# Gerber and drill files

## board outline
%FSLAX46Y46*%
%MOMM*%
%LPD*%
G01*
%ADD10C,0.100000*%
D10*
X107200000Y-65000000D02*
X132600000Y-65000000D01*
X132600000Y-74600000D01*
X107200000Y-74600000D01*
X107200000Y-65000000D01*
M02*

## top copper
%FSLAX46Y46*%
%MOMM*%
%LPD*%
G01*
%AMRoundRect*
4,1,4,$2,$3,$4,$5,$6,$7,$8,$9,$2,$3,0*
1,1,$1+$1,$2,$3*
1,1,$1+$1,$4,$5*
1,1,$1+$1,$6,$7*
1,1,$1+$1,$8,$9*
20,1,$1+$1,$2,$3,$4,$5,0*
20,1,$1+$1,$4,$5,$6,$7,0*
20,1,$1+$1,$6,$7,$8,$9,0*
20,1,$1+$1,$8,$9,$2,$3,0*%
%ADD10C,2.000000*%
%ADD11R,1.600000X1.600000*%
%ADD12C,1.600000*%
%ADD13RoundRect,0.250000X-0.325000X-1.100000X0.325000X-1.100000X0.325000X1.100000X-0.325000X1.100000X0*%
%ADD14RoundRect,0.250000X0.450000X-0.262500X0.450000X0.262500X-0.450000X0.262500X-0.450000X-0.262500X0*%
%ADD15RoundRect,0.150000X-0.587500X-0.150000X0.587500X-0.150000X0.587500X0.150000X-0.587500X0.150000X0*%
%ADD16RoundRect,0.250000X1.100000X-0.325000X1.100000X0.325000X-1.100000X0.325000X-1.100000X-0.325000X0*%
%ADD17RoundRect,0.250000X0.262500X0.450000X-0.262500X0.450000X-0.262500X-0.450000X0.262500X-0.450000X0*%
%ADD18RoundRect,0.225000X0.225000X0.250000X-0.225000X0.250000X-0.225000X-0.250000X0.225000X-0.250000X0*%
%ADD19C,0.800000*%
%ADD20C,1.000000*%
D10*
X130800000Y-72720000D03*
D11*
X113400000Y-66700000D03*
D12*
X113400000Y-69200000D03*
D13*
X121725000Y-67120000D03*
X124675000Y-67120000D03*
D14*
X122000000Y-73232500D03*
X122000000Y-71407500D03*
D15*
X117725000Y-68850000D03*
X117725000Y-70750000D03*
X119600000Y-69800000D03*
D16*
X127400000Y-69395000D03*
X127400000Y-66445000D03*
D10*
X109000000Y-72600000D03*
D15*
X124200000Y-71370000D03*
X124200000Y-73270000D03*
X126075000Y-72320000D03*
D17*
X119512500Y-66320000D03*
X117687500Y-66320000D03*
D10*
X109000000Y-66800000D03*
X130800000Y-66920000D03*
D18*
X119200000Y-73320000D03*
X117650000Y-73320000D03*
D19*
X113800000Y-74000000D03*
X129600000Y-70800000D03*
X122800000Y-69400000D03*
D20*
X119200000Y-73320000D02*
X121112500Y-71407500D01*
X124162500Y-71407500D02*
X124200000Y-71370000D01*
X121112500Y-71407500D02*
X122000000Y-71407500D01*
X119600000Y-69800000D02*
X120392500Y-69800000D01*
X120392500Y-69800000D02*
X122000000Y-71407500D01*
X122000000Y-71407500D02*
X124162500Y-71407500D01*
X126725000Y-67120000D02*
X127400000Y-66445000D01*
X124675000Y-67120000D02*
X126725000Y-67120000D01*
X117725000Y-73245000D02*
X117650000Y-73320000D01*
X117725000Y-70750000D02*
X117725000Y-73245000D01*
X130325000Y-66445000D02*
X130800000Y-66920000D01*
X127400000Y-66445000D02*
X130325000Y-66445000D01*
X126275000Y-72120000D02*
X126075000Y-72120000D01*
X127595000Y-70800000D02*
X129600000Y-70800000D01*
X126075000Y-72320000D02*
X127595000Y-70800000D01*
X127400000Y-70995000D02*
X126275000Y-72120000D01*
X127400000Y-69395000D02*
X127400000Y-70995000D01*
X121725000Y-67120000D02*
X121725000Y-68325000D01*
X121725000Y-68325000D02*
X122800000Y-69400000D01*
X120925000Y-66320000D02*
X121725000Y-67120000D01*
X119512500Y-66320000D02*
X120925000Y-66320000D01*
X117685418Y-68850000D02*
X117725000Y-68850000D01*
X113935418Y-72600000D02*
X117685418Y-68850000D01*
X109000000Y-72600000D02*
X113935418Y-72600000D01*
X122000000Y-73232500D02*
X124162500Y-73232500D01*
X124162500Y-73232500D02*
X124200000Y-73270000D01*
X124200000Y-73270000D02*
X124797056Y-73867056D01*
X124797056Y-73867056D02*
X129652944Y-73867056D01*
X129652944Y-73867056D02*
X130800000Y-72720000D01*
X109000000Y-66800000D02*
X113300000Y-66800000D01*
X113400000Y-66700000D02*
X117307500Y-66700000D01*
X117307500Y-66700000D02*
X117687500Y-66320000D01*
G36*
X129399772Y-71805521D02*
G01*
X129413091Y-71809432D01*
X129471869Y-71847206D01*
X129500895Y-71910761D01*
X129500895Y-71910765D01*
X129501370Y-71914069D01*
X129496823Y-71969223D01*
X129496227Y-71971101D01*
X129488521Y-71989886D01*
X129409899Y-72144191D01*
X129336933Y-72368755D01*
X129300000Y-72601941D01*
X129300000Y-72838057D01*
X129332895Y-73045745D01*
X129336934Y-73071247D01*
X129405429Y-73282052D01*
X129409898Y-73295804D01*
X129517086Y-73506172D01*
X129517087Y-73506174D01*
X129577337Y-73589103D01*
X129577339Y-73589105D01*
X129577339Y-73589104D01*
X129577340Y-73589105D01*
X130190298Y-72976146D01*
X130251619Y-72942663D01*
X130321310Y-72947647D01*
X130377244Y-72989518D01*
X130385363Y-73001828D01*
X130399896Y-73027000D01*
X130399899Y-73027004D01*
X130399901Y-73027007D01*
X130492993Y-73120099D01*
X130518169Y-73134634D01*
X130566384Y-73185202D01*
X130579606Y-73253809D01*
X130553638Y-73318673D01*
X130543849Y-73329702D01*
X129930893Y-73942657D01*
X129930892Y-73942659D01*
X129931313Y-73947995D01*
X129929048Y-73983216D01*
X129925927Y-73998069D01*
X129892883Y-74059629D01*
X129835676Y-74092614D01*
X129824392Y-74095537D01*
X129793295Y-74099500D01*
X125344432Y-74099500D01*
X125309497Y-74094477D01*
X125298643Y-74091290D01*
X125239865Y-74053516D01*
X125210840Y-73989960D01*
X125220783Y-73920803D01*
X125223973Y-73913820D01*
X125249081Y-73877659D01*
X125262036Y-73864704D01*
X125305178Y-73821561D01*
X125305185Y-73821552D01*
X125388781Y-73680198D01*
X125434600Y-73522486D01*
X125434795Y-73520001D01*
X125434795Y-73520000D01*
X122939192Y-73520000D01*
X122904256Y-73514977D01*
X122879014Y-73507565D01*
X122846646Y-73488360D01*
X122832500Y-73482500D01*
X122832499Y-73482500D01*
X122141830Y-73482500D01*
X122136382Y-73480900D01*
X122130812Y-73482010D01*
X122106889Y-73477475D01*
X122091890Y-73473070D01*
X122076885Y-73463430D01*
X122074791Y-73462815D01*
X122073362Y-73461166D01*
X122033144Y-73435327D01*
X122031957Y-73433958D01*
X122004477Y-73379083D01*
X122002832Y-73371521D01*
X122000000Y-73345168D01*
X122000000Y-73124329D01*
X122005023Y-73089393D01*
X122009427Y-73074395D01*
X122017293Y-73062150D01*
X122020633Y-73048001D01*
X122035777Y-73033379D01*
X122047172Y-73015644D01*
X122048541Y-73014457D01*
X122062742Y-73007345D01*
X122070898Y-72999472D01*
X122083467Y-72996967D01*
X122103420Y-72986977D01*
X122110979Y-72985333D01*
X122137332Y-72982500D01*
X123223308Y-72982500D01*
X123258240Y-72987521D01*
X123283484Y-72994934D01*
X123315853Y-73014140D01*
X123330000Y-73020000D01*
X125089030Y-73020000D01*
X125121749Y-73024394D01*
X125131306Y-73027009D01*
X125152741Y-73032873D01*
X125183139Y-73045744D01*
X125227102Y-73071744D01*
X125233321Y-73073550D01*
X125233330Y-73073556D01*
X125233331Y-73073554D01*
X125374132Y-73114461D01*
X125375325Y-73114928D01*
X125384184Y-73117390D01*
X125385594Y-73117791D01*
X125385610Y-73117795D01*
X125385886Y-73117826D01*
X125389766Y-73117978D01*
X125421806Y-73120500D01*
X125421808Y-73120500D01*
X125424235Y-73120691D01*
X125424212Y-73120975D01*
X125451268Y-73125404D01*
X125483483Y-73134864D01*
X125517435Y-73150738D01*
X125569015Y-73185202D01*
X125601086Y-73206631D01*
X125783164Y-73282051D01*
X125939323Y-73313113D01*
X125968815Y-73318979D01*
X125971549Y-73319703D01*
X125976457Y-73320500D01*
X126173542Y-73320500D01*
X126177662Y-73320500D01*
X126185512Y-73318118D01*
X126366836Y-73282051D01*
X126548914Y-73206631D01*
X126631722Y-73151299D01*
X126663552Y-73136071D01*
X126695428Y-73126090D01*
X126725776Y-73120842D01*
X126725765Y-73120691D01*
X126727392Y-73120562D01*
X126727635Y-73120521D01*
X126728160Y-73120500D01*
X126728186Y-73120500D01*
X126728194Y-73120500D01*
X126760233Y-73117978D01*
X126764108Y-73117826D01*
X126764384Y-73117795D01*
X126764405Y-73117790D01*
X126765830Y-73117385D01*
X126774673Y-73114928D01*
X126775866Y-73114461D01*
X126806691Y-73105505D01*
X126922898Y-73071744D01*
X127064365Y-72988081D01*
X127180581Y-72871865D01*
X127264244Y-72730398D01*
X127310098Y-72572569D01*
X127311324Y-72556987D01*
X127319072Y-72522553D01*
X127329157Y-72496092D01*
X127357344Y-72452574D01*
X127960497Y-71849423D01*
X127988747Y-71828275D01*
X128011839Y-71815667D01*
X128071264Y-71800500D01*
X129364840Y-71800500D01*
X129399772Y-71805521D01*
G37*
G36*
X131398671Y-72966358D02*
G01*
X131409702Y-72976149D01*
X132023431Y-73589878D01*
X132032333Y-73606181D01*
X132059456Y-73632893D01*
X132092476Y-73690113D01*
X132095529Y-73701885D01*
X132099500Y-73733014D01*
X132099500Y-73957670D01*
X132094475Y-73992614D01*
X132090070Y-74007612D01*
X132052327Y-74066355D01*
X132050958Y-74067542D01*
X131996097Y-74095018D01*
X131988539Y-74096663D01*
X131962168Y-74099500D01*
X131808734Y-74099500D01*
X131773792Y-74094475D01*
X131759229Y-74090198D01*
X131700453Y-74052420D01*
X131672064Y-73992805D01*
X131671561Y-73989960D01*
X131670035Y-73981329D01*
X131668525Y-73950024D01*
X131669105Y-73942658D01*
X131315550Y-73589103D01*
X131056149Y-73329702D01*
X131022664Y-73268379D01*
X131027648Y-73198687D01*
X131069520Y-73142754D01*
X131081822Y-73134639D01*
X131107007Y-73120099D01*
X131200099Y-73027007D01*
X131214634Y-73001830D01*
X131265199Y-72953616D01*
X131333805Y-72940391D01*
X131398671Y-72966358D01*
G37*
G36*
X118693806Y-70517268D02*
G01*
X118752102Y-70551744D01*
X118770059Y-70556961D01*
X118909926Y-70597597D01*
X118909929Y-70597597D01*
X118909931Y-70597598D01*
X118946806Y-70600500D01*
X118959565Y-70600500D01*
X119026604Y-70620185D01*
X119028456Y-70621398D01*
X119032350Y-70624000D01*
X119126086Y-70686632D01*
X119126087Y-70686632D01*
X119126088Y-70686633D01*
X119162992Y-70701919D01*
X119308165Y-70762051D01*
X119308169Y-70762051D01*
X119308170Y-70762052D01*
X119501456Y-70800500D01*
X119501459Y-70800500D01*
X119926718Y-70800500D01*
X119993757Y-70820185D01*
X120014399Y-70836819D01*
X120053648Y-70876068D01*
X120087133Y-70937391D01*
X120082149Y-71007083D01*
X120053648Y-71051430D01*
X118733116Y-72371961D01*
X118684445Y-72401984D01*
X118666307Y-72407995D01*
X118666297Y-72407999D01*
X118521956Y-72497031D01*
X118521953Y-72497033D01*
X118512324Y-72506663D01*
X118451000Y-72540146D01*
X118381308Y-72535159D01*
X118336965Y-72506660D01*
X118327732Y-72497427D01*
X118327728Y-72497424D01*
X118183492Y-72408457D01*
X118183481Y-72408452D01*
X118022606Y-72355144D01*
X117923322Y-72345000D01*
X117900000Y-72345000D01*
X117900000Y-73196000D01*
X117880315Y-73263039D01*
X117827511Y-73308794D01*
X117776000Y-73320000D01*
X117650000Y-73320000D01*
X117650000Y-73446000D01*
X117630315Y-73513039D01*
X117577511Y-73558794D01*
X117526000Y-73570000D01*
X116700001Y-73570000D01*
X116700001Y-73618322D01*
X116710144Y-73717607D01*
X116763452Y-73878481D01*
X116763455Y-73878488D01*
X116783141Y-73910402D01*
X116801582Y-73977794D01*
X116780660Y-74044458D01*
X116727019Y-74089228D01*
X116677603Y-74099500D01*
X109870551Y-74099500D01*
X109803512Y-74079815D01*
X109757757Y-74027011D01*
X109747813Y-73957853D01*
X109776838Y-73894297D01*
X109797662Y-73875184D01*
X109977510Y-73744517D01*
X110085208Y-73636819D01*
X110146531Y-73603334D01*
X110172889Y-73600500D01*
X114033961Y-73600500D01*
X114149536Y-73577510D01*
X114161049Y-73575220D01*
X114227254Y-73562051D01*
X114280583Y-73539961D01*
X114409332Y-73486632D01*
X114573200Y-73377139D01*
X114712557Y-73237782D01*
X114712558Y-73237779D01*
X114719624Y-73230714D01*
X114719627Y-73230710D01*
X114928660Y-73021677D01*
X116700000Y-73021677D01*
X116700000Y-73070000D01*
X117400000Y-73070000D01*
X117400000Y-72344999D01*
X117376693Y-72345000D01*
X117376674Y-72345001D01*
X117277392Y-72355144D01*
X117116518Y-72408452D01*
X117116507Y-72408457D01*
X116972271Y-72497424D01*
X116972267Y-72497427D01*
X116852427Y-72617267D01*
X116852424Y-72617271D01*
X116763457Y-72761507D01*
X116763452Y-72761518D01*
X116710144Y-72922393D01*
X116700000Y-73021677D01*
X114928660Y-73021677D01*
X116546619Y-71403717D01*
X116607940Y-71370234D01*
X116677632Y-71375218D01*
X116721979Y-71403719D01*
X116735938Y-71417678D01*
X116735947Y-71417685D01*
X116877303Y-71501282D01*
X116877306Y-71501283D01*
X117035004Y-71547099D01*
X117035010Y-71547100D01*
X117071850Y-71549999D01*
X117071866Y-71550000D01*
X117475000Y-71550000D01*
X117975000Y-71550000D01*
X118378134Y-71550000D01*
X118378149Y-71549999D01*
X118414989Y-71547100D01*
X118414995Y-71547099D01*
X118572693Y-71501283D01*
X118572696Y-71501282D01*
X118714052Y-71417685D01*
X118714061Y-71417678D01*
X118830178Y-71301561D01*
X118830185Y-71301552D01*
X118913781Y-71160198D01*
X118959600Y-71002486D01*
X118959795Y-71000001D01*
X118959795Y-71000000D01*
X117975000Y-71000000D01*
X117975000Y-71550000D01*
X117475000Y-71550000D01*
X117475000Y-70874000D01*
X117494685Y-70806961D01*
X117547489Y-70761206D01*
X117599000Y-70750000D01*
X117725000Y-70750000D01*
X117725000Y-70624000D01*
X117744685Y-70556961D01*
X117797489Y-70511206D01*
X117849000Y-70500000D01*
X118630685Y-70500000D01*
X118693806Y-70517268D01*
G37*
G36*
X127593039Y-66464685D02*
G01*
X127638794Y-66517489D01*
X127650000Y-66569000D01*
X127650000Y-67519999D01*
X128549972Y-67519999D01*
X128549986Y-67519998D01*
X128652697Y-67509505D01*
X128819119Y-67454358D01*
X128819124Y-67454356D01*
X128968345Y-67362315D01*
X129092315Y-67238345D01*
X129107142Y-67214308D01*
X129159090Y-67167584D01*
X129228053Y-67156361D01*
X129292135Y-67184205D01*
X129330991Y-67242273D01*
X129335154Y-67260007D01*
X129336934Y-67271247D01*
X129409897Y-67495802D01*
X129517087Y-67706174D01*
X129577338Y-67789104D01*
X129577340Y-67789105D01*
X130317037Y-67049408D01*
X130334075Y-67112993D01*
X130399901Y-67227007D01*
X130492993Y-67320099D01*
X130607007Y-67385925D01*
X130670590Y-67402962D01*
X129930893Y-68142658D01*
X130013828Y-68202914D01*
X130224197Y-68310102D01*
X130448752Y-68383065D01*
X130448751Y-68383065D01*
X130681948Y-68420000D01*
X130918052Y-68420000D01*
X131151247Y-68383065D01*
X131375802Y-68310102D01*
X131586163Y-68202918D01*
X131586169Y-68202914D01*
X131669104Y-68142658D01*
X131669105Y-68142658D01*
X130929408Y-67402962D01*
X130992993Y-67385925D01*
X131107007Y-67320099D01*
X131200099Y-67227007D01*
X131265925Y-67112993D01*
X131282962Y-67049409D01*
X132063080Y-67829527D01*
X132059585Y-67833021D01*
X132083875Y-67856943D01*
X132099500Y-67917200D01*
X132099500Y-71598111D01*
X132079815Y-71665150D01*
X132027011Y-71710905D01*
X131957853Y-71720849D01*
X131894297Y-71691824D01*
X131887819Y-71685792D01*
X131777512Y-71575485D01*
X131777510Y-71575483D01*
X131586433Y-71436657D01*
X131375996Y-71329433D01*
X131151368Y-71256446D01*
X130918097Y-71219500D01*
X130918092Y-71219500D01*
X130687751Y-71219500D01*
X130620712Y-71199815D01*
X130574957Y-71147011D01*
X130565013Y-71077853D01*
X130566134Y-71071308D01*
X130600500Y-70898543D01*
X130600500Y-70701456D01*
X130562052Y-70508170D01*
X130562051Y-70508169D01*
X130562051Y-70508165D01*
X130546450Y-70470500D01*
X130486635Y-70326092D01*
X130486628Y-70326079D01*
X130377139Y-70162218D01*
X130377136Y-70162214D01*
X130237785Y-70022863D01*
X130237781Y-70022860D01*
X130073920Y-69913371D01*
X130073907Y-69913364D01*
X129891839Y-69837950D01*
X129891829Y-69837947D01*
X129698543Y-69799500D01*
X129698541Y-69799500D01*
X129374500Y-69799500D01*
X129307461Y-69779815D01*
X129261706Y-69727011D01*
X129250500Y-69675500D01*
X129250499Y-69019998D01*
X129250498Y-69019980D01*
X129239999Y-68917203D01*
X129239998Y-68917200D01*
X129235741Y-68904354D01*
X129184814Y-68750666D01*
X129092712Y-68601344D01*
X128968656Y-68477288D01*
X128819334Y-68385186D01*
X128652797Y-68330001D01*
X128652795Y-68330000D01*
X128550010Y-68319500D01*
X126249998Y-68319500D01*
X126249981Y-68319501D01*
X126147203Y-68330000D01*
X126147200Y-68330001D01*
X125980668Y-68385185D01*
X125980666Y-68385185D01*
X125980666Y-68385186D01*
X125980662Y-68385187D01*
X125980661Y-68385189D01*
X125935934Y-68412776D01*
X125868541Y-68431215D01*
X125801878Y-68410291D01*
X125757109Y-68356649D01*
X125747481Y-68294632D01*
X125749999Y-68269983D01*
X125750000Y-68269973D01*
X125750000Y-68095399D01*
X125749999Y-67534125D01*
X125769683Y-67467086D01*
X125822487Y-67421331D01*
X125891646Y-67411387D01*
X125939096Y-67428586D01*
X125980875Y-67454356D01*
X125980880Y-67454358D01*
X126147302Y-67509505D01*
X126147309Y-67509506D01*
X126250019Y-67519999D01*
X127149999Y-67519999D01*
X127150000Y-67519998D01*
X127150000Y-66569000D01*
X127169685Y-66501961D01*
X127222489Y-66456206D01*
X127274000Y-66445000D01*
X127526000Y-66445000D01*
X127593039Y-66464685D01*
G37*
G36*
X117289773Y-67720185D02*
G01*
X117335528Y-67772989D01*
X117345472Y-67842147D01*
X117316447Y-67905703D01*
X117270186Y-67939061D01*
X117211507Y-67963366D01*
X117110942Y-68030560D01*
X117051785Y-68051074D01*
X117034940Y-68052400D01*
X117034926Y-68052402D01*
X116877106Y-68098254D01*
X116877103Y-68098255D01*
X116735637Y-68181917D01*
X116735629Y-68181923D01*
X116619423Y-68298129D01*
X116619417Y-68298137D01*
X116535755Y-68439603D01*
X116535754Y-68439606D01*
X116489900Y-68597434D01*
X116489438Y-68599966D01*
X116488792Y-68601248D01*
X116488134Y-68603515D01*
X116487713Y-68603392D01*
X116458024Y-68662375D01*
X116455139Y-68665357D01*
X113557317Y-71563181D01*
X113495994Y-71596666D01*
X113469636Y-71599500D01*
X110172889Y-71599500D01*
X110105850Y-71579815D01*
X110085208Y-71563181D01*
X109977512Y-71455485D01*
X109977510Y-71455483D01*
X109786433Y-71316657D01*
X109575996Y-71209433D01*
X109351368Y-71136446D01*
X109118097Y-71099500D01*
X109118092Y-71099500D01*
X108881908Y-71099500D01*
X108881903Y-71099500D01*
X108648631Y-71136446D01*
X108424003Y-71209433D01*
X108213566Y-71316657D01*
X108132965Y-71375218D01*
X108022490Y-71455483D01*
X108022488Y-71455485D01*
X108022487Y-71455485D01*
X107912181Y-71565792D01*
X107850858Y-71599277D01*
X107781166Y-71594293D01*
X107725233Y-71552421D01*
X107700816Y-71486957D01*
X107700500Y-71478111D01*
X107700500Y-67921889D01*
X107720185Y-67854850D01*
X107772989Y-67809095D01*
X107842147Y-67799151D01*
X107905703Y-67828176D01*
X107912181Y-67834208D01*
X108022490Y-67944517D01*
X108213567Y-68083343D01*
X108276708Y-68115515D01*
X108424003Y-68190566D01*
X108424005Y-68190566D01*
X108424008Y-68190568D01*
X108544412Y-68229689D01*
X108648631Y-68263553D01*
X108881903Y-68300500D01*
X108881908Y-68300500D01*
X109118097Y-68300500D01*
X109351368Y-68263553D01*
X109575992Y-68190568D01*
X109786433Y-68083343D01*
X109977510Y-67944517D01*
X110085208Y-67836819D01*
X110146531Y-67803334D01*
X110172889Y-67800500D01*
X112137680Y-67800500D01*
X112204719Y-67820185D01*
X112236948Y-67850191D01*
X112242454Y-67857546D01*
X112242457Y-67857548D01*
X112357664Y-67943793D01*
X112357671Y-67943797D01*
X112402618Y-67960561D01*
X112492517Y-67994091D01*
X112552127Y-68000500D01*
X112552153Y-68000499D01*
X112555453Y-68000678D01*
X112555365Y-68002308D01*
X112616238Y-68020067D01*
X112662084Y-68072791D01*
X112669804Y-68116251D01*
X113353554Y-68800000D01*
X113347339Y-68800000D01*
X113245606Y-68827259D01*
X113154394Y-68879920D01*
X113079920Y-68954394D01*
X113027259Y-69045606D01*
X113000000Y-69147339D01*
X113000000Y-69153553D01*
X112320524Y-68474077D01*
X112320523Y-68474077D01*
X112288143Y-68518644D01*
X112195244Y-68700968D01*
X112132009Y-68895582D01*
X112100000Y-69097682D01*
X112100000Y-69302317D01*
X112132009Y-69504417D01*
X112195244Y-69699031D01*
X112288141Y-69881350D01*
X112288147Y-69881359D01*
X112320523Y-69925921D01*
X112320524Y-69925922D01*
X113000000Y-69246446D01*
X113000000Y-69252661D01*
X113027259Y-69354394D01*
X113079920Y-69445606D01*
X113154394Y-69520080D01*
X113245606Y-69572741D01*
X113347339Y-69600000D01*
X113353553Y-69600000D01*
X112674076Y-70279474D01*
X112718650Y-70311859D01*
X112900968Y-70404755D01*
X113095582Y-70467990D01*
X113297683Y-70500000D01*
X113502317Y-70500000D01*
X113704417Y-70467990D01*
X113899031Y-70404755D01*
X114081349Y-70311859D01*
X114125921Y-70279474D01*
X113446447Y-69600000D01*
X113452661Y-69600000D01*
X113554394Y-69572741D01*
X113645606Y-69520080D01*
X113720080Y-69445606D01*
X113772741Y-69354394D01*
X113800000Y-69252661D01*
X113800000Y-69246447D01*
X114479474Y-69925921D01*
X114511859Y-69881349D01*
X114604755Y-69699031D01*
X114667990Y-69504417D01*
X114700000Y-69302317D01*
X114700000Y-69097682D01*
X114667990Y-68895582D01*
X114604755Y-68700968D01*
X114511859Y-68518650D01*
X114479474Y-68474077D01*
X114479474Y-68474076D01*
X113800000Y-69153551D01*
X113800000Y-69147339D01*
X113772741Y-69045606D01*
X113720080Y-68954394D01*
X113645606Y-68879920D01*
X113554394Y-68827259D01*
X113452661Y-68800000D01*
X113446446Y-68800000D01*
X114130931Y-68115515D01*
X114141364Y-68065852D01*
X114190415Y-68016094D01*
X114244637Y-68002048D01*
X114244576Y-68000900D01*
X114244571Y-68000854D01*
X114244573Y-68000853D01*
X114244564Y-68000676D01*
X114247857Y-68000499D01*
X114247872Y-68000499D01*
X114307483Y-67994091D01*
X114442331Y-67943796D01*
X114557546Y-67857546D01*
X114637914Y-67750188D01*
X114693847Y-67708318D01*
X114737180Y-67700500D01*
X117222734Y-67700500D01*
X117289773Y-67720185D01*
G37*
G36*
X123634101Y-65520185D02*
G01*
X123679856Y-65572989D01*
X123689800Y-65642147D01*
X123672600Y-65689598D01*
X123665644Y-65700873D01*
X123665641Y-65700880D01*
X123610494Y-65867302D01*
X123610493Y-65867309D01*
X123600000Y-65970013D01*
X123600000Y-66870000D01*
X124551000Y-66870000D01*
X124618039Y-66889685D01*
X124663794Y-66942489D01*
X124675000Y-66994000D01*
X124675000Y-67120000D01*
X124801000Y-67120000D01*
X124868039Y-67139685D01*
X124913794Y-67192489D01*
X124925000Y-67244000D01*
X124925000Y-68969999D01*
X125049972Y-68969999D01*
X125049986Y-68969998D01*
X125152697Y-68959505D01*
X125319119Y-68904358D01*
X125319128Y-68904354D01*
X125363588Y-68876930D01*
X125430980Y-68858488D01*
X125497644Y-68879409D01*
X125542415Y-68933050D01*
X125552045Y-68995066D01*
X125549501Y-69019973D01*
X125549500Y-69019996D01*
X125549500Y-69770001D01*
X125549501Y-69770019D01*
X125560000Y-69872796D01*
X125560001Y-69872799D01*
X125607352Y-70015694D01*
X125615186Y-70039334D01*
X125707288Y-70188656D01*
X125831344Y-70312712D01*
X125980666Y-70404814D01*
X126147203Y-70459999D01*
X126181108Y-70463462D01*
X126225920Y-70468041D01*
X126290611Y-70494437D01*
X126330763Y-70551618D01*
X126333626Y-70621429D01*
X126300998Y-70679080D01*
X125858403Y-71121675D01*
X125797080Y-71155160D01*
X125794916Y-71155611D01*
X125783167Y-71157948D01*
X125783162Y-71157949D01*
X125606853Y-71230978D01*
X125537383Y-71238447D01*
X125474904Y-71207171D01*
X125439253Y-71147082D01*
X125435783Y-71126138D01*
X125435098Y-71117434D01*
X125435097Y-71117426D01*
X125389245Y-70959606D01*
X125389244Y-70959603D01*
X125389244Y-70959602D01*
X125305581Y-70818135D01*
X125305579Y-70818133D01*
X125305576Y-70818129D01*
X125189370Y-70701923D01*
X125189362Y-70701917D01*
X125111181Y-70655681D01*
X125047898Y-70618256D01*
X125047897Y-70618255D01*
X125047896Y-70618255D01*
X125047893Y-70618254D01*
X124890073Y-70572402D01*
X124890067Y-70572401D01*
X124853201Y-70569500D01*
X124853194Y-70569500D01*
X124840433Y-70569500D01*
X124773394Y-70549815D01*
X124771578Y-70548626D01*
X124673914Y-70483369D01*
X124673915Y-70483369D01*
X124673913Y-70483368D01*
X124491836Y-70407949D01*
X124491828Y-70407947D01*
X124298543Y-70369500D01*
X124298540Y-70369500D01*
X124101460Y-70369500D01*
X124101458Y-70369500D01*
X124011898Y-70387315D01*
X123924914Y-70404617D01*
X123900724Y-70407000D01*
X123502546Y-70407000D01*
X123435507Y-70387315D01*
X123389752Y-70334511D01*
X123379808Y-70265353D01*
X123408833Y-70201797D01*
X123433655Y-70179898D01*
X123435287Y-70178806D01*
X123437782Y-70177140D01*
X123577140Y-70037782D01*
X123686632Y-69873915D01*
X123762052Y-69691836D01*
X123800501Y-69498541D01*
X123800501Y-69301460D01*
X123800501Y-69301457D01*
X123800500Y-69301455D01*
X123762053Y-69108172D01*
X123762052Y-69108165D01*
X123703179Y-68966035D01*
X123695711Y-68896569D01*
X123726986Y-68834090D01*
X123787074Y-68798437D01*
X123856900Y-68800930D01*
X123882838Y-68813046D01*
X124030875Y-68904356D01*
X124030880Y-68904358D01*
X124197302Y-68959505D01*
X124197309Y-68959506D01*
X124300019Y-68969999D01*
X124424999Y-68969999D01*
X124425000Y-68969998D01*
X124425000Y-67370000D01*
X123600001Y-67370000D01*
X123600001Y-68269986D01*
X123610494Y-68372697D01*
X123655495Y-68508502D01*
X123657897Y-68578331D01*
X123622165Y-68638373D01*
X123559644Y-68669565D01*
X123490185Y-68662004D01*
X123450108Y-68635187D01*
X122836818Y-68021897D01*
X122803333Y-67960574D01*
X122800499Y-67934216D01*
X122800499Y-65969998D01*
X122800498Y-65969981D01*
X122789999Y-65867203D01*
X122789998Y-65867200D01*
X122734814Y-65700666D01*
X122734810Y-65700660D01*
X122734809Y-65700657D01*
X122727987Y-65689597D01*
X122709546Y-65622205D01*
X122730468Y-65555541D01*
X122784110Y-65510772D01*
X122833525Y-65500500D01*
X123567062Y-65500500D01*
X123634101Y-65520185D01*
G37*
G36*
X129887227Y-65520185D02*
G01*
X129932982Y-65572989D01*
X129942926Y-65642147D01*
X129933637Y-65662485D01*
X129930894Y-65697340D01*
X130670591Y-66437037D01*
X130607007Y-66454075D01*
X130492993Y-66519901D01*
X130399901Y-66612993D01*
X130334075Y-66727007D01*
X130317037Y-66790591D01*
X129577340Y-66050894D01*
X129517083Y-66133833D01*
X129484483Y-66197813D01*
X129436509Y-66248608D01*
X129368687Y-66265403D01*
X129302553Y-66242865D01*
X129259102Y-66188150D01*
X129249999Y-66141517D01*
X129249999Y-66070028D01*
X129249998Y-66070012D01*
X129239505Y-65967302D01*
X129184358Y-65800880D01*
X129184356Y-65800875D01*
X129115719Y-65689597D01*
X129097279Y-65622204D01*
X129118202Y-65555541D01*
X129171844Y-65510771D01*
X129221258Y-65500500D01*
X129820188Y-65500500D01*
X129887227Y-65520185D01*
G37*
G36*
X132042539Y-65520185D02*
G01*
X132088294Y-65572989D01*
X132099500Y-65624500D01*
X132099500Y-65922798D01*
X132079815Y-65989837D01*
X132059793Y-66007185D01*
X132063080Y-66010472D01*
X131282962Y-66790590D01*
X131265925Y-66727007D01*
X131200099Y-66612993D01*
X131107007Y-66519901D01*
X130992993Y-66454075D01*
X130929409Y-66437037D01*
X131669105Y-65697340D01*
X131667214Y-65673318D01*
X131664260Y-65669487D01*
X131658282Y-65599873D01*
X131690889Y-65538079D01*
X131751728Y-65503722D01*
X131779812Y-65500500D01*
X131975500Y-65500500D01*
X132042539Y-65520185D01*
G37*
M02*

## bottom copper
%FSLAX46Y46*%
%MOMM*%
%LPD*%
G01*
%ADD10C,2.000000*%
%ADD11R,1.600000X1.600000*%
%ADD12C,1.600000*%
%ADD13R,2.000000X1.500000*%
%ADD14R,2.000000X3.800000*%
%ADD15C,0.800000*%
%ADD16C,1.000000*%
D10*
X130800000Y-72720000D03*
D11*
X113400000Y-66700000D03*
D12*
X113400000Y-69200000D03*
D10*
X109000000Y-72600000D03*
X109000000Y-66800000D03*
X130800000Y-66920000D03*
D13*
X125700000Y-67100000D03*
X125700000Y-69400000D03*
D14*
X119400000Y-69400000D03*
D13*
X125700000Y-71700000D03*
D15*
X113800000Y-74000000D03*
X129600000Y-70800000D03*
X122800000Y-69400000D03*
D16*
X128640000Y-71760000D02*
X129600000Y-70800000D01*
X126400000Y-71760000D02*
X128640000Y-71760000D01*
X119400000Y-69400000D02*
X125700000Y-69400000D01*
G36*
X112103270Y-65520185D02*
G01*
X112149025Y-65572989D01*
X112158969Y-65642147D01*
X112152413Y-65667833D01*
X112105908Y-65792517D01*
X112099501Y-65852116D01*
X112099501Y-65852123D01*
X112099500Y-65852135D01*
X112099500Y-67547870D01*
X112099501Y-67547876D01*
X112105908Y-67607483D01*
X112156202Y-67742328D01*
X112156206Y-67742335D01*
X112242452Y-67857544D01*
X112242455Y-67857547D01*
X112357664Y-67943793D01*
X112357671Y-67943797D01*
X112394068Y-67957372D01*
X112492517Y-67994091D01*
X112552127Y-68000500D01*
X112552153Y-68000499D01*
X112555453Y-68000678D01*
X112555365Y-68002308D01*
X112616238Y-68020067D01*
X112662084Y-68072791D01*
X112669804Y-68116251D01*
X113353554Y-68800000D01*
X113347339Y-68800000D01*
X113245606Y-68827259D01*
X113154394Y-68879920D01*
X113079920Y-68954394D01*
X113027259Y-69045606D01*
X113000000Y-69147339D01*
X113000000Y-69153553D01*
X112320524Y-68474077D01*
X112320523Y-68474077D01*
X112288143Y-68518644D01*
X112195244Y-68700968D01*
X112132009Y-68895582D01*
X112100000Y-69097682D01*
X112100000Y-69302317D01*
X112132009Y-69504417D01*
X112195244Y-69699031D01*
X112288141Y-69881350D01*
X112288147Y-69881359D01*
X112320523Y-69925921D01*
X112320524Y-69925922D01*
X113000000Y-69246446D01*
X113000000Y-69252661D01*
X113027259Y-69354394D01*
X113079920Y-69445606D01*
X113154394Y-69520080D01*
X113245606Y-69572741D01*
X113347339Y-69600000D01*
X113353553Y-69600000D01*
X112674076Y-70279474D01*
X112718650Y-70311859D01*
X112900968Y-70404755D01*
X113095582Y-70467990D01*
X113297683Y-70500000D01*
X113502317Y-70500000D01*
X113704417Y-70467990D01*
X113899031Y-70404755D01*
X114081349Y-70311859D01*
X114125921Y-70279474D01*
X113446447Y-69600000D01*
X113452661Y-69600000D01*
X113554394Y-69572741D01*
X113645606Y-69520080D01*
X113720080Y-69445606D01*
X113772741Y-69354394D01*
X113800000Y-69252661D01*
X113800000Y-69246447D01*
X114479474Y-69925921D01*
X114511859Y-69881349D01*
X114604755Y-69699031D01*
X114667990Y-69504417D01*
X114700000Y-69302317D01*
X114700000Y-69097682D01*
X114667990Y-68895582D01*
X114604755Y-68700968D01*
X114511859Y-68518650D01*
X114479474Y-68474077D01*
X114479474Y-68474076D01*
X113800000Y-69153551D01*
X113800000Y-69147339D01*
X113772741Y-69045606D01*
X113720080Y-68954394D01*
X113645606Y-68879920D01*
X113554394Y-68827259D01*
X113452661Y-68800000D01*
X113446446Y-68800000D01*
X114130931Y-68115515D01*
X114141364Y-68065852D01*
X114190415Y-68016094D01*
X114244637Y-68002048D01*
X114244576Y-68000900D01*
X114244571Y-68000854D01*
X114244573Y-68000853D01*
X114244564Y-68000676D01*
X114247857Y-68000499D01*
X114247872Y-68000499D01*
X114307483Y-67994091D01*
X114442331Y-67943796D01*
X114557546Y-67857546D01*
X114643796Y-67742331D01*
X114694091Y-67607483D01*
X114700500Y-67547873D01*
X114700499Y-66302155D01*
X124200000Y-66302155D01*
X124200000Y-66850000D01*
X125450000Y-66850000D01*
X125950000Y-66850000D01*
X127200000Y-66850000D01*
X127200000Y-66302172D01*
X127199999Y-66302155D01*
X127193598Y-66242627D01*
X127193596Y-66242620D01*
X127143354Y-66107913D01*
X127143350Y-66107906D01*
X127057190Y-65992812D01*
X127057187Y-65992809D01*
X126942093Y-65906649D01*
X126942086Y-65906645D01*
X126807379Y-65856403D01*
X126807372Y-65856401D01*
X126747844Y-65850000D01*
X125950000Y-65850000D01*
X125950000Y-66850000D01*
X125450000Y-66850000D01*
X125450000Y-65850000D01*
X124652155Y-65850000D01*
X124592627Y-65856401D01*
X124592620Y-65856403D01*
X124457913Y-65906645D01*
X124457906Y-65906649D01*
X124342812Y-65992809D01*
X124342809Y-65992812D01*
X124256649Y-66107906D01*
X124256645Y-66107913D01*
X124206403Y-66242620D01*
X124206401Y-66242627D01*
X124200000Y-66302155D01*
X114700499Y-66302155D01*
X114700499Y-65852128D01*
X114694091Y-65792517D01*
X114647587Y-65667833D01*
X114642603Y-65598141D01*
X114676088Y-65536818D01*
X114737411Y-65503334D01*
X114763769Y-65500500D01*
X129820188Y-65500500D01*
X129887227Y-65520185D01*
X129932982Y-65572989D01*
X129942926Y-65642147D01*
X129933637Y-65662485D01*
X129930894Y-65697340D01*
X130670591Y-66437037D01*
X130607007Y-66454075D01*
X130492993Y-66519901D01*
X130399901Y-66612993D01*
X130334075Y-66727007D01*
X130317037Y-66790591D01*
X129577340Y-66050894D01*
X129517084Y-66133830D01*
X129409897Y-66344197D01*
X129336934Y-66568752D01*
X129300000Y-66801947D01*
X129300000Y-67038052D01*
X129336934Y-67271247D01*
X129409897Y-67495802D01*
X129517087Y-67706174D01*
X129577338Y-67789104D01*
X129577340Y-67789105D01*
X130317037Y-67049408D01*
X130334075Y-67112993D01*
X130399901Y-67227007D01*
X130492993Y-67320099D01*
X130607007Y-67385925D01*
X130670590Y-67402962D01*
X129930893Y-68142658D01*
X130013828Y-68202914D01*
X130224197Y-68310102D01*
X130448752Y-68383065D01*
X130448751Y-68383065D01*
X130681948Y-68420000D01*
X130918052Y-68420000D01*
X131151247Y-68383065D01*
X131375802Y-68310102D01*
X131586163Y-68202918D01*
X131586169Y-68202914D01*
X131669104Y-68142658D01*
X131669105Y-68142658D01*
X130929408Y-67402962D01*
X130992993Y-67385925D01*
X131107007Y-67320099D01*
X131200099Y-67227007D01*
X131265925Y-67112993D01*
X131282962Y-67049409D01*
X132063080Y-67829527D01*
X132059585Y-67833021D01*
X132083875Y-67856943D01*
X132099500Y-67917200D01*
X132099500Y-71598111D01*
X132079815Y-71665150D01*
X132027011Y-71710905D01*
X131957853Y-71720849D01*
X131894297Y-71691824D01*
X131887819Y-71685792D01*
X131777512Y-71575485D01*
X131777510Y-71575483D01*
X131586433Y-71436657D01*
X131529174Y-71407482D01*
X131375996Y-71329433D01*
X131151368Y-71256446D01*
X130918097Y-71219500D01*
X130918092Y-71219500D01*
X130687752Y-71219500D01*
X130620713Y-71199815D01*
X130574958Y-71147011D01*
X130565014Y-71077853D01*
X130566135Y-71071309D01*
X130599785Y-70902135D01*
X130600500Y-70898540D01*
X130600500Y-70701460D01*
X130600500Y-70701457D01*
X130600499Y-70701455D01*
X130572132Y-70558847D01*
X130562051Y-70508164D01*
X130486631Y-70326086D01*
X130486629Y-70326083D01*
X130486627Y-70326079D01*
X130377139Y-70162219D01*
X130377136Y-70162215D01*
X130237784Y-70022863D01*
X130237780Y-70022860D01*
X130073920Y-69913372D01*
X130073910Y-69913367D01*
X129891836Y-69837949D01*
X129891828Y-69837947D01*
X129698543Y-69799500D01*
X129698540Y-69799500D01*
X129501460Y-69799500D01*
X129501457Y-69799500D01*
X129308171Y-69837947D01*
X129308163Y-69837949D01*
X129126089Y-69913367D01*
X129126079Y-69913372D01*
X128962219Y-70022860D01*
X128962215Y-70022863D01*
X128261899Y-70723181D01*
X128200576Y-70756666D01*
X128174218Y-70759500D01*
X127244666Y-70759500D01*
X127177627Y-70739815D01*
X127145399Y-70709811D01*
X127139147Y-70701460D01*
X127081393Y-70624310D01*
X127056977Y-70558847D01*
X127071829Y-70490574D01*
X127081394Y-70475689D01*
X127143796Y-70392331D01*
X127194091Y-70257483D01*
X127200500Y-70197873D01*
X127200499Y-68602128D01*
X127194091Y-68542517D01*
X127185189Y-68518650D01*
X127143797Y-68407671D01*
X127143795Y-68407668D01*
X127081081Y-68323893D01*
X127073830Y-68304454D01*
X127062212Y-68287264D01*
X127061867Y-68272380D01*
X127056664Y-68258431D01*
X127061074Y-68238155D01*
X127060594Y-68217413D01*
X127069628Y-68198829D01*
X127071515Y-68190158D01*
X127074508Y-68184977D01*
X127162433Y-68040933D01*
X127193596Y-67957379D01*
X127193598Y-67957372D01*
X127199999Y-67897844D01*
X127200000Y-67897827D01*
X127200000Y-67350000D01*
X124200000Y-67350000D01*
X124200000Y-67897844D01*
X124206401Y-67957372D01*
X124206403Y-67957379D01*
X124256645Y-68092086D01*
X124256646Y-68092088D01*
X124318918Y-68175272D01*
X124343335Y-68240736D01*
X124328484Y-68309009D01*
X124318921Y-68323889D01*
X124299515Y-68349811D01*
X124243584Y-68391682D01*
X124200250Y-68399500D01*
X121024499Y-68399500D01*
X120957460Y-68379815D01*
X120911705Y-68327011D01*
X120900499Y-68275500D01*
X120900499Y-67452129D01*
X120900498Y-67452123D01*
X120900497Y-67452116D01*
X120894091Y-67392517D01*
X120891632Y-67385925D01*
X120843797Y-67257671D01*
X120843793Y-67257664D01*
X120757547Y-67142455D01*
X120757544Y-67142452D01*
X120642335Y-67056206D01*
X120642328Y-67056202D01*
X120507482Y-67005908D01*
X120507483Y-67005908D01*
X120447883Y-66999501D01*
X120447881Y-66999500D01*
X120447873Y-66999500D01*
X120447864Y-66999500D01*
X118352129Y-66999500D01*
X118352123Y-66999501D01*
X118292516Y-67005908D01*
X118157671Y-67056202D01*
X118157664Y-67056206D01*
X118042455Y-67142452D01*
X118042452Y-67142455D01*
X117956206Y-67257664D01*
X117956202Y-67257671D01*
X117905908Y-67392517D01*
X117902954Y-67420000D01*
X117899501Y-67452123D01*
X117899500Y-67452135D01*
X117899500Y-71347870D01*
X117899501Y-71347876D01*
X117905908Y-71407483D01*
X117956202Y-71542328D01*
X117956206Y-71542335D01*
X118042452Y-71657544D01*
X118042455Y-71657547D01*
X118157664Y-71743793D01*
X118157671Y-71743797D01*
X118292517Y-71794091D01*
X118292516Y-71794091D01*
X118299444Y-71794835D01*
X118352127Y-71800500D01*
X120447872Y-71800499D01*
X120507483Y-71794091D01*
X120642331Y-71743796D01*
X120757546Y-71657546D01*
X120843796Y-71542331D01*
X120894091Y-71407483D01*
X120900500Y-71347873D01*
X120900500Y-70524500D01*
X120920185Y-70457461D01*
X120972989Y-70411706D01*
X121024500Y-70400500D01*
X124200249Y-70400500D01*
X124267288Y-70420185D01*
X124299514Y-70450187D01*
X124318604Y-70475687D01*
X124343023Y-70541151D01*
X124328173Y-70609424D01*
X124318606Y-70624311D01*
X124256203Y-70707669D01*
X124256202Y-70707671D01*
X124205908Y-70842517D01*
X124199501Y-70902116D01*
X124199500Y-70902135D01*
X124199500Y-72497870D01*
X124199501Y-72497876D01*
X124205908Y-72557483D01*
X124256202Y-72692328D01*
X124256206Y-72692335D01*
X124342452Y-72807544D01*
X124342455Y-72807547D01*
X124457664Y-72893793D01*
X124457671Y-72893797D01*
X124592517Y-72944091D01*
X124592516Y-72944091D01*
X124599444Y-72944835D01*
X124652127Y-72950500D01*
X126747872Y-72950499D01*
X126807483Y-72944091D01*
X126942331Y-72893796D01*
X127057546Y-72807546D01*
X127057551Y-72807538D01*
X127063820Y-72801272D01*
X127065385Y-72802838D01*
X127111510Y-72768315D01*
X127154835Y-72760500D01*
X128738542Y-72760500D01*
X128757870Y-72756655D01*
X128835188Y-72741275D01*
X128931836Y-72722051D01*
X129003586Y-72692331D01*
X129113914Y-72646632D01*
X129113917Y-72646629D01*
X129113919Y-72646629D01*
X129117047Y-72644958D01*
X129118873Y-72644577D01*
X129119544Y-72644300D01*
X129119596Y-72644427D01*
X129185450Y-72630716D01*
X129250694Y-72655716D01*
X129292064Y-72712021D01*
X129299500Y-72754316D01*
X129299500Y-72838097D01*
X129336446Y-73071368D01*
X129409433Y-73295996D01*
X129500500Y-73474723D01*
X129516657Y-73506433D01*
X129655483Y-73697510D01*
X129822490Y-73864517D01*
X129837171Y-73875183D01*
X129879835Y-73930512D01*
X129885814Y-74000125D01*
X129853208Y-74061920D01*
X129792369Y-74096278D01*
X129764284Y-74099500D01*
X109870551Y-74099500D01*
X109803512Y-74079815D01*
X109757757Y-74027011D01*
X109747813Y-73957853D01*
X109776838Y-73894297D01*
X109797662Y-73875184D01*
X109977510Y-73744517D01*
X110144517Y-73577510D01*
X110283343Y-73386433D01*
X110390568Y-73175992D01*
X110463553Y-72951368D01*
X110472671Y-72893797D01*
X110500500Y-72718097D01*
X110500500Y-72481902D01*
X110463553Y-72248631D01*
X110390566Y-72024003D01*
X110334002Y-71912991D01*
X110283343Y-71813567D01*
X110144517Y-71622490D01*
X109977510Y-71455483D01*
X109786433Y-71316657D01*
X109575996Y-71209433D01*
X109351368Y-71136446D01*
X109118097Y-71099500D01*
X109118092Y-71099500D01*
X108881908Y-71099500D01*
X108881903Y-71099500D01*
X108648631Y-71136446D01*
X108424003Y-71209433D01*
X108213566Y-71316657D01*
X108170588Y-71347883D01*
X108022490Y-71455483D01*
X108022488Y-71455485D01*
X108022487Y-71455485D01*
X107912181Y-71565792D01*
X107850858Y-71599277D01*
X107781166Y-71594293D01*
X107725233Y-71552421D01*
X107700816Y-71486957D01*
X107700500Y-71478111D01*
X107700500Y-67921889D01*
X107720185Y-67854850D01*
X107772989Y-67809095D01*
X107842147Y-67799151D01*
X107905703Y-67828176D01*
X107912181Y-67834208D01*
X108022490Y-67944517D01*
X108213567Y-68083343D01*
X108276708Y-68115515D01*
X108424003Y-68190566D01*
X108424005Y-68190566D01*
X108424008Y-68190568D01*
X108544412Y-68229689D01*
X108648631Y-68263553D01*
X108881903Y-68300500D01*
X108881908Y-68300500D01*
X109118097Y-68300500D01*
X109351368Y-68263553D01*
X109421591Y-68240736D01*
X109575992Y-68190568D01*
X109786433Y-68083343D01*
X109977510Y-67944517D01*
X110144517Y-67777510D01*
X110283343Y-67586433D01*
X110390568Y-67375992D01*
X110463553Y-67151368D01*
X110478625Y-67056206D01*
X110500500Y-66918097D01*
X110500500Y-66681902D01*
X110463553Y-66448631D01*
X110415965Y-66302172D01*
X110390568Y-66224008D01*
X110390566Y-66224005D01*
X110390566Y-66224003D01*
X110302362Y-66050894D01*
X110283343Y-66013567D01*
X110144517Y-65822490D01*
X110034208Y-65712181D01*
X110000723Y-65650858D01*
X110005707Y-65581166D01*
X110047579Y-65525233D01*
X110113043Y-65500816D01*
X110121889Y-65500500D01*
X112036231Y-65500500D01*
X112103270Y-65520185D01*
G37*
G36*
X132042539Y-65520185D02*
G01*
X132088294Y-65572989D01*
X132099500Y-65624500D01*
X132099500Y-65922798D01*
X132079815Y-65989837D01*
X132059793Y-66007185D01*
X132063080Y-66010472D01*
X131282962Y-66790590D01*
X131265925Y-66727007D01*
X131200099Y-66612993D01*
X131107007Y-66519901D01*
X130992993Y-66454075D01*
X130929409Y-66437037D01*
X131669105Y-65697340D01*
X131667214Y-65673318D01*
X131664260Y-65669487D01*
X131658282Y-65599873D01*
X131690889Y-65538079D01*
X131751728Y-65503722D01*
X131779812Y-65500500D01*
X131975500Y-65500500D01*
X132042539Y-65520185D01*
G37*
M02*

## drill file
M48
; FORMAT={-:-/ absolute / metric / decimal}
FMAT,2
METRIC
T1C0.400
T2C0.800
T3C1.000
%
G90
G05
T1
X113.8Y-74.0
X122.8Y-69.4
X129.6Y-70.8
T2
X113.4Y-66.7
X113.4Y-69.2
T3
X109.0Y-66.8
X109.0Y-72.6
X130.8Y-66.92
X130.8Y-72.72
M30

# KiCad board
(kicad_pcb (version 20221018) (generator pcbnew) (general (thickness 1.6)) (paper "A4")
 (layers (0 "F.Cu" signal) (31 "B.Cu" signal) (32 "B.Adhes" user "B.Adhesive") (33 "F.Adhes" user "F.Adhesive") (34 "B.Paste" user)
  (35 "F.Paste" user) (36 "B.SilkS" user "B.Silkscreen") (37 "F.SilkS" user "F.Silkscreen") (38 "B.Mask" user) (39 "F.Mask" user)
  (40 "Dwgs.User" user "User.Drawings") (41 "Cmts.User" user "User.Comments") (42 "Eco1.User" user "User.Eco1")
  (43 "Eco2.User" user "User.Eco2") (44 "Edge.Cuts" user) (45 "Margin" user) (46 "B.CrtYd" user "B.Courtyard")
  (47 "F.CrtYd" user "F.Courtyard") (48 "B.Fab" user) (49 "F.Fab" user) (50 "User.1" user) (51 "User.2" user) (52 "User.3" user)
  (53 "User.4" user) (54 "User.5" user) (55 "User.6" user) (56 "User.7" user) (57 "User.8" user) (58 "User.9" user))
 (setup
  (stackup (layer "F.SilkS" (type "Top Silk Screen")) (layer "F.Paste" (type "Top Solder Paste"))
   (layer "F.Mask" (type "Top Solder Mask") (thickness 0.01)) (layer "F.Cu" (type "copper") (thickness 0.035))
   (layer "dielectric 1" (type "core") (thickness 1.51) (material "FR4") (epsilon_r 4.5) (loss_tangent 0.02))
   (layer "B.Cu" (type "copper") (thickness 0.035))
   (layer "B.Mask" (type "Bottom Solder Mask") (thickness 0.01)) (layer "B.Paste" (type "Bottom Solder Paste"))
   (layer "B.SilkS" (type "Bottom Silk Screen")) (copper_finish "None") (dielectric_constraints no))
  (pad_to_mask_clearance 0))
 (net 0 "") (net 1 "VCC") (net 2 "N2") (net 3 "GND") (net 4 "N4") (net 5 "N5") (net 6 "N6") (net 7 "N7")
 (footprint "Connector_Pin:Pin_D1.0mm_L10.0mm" (layer "F.Cu") (at 130.8 72.72)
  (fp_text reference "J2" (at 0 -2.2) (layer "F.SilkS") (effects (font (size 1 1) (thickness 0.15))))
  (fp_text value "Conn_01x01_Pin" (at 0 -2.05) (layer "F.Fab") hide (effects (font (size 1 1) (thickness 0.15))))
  (pad "1" thru_hole circle (at 0 0) (size 2 2) (drill 1) (layers "*.Cu" "*.Mask") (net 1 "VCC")))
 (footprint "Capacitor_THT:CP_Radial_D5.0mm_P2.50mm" (layer "F.Cu") (at 113.4 66.7 -90)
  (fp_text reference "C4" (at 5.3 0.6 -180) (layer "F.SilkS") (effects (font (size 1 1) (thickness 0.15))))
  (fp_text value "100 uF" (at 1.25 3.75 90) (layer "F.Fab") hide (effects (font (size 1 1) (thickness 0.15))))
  (pad "1" thru_hole rect (at 0 0 270) (size 1.6 1.6) (drill 0.8) (layers "*.Cu" "*.Mask") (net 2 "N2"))
  (pad "2" thru_hole circle (at 2.5 0 270) (size 1.6 1.6) (drill 0.8) (layers "*.Cu" "*.Mask") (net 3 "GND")))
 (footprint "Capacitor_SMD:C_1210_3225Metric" (layer "F.Cu") (at 123.2 67.12)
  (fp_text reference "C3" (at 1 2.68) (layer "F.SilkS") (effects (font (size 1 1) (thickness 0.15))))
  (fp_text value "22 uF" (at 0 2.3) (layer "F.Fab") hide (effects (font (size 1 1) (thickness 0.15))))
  (pad "1" smd roundrect (at -1.475 0) (size 1.15 2.7) (layers "F.Cu" "F.Paste" "F.Mask") (roundrect_rratio 0.2173913043) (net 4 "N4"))
  (pad "2" smd roundrect (at 1.475 0) (size 1.15 2.7) (layers "F.Cu" "F.Paste" "F.Mask") (roundrect_rratio 0.2173913043) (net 3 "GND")))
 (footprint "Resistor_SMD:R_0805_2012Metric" (layer "F.Cu") (at 122 72.32 90)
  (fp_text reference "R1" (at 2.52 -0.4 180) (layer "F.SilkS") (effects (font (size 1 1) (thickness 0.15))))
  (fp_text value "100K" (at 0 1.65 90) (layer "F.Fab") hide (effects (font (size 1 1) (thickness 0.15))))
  (pad "1" smd roundrect (at -0.9125 0 90) (size 1.025 1.4) (layers "F.Cu" "F.Paste" "F.Mask") (roundrect_rratio 0.243902439) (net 1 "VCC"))
  (pad "2" smd roundrect (at 0.9125 0 90) (size 1.025 1.4) (layers "F.Cu" "F.Paste" "F.Mask") (roundrect_rratio 0.243902439) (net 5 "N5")))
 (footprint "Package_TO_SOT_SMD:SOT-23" (layer "F.Cu") (at 118.6625 69.8)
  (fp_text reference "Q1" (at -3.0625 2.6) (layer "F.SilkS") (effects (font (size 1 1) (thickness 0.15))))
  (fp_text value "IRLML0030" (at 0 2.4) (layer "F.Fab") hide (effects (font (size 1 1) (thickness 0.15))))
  (pad "1" smd roundrect (at -0.9375 -0.95) (size 1.475 0.6) (layers "F.Cu" "F.Paste" "F.Mask") (roundrect_rratio 0.25) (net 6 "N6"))
  (pad "2" smd roundrect (at -0.9375 0.95) (size 1.475 0.6) (layers "F.Cu" "F.Paste" "F.Mask") (roundrect_rratio 0.25) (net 3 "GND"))
  (pad "3" smd roundrect (at 0.9375 0) (size 1.475 0.6) (layers "F.Cu" "F.Paste" "F.Mask") (roundrect_rratio 0.25) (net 5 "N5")))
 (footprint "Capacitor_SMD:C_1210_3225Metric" (layer "F.Cu") (at 127.4 67.92 90)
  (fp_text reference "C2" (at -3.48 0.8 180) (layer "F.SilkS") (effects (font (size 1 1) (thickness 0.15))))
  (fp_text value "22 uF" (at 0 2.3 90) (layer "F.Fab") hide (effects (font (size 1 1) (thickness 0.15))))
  (pad "1" smd roundrect (at -1.475 0 90) (size 1.15 2.7) (layers "F.Cu" "F.Paste" "F.Mask") (roundrect_rratio 0.2173913043) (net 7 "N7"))
  (pad "2" smd roundrect (at 1.475 0 90) (size 1.15 2.7) (layers "F.Cu" "F.Paste" "F.Mask") (roundrect_rratio 0.2173913043) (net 3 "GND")))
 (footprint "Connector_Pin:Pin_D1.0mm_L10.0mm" (layer "F.Cu") (at 109 72.6)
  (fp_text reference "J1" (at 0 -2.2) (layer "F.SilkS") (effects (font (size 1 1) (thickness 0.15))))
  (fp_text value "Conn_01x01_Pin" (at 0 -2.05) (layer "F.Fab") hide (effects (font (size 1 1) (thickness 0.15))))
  (pad "1" thru_hole circle (at 0 0) (size 2 2) (drill 1) (layers "*.Cu" "*.Mask") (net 6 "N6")))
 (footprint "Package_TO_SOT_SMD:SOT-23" (layer "F.Cu") (at 125.1375 72.32)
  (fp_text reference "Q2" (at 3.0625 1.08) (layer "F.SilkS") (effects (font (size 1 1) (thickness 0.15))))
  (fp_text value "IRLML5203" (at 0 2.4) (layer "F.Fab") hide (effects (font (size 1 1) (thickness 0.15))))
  (pad "1" smd roundrect (at -0.9375 -0.95) (size 1.475 0.6) (layers "F.Cu" "F.Paste" "F.Mask") (roundrect_rratio 0.25) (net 5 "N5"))
  (pad "2" smd roundrect (at -0.9375 0.95) (size 1.475 0.6) (layers "F.Cu" "F.Paste" "F.Mask") (roundrect_rratio 0.25) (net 1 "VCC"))
  (pad "3" smd roundrect (at 0.9375 0) (size 1.475 0.6) (layers "F.Cu" "F.Paste" "F.Mask") (roundrect_rratio 0.25) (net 7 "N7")))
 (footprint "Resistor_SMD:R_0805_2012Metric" (layer "F.Cu") (at 118.6 66.32 180)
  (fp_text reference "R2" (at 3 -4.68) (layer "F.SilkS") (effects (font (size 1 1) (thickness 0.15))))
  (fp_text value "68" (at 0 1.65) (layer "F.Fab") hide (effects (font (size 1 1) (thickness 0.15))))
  (pad "1" smd roundrect (at -0.9125 0 180) (size 1.025 1.4) (layers "F.Cu" "F.Paste" "F.Mask") (roundrect_rratio 0.243902439) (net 4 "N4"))
  (pad "2" smd roundrect (at 0.9125 0 180) (size 1.025 1.4) (layers "F.Cu" "F.Paste" "F.Mask") (roundrect_rratio 0.243902439) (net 2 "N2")))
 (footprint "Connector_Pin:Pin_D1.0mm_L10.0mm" (layer "F.Cu") (at 109 66.8)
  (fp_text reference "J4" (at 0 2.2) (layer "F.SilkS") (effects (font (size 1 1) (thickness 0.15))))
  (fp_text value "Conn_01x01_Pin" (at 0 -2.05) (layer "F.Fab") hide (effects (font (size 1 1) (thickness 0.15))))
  (pad "1" thru_hole circle (at 0 0) (size 2 2) (drill 1) (layers "*.Cu" "*.Mask") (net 2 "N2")))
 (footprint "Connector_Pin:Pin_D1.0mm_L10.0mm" (layer "F.Cu") (at 130.8 66.92)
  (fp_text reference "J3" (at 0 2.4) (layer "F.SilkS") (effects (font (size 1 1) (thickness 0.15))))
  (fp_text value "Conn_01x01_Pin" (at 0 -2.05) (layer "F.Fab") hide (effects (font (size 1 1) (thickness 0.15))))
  (pad "1" thru_hole circle (at 0 0) (size 2 2) (drill 1) (layers "*.Cu" "*.Mask") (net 3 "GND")))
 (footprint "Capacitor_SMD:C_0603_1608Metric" (layer "F.Cu") (at 118.425 73.32 180)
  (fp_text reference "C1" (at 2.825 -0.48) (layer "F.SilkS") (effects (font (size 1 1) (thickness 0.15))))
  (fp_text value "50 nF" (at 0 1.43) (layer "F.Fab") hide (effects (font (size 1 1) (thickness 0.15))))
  (pad "1" smd roundrect (at -0.775 0 180) (size 0.9 0.95) (layers "F.Cu" "F.Paste" "F.Mask") (roundrect_rratio 0.25) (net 5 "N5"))
  (pad "2" smd roundrect (at 0.775 0 180) (size 0.9 0.95) (layers "F.Cu" "F.Paste" "F.Mask") (roundrect_rratio 0.25) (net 3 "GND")))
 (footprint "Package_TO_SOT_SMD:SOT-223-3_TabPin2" (layer "B.Cu") (at 122.55 69.4 180)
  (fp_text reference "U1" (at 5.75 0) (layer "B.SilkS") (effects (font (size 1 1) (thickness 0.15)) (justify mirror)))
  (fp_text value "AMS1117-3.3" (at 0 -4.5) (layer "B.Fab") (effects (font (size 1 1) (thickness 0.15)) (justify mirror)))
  (pad "1" smd rect (at -3.15 2.3 180) (size 2 1.5) (layers "B.Cu" "B.Paste" "B.Mask") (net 3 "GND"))
  (pad "2" smd rect (at -3.15 0 180) (size 2 1.5) (layers "B.Cu" "B.Paste" "B.Mask") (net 4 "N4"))
  (pad "2" smd rect (at 3.15 0 180) (size 2 3.8) (layers "B.Cu" "B.Paste" "B.Mask") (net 4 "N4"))
  (pad "3" smd rect (at -3.15 -2.3 180) (size 2 1.5) (layers "B.Cu" "B.Paste" "B.Mask") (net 7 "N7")))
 (gr_rect (start 107.2 65) (end 132.6 74.6) (stroke (width 0.1) (type default)) (fill none) (layer "Edge.Cuts"))
 (segment (start 119.2 73.32) (end 121.1125 71.4075) (width 1) (layer "F.Cu") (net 5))
 (segment (start 124.1625 71.4075) (end 124.2 71.37) (width 1) (layer "F.Cu") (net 5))
 (segment (start 121.1125 71.4075) (end 122 71.4075) (width 1) (layer "F.Cu") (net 5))
 (segment (start 119.6 69.8) (end 120.3925 69.8) (width 1) (layer "F.Cu") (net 5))
 (segment (start 120.3925 69.8) (end 122 71.4075) (width 1) (layer "F.Cu") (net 5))
 (segment (start 122 71.4075) (end 124.1625 71.4075) (width 1) (layer "F.Cu") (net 5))
 (segment (start 126.725 67.12) (end 127.4 66.445) (width 1) (layer "F.Cu") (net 3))
 (segment (start 124.675 67.12) (end 126.725 67.12) (width 1) (layer "F.Cu") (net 3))
 (segment (start 117.725 73.245) (end 117.65 73.32) (width 1) (layer "F.Cu") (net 3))
 (segment (start 117.725 70.75) (end 117.725 73.245) (width 1) (layer "F.Cu") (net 3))
 (segment (start 130.325 66.445) (end 130.8 66.92) (width 1) (layer "F.Cu") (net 3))
 (segment (start 127.4 66.445) (end 130.325 66.445) (width 1) (layer "F.Cu") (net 3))
 (via (at 113.8 74) (size 0.8) (drill 0.4) (layers "F.Cu" "B.Cu") (free) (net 3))
 (segment (start 126.275 72.12) (end 126.075 72.12) (width 1) (layer "F.Cu") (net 7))
 (segment (start 127.595 70.8) (end 129.6 70.8) (width 1) (layer "F.Cu") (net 7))
 (segment (start 126.075 72.32) (end 127.595 70.8) (width 1) (layer "F.Cu") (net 7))
 (segment (start 127.4 70.995) (end 126.275 72.12) (width 1) (layer "F.Cu") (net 7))
 (segment (start 127.4 69.395) (end 127.4 70.995) (width 1) (layer "F.Cu") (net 7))
 (via (at 129.6 70.8) (size 0.8) (drill 0.4) (layers "F.Cu" "B.Cu") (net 7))
 (segment (start 128.64 71.76) (end 129.6 70.8) (width 1) (layer "B.Cu") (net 7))
 (segment (start 126.4 71.76) (end 128.64 71.76) (width 1) (layer "B.Cu") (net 7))
 (segment (start 121.725 67.12) (end 121.725 68.325) (width 1) (layer "F.Cu") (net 4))
 (segment (start 121.725 68.325) (end 122.8 69.4) (width 1) (layer "F.Cu") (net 4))
 (segment (start 120.925 66.32) (end 121.725 67.12) (width 1) (layer "F.Cu") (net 4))
 (segment (start 119.5125 66.32) (end 120.925 66.32) (width 1) (layer "F.Cu") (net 4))
 (via (at 122.8 69.4) (size 0.8) (drill 0.4) (layers "F.Cu" "B.Cu") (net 4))
 (segment (start 119.4 69.4) (end 125.7 69.4) (width 1) (layer "B.Cu") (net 4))
 (segment (start 117.685418 68.85) (end 117.725 68.85) (width 1) (layer "F.Cu") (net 6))
 (segment (start 113.935418 72.6) (end 117.685418 68.85) (width 1) (layer "F.Cu") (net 6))
 (segment (start 109 72.6) (end 113.935418 72.6) (width 1) (layer "F.Cu") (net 6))
 (segment (start 122 73.2325) (end 124.1625 73.2325) (width 1) (layer "F.Cu") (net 1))
 (segment (start 124.1625 73.2325) (end 124.2 73.27) (width 1) (layer "F.Cu") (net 1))
 (segment (start 124.2 73.27) (end 124.797056 73.867056) (width 1) (layer "F.Cu") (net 1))
 (segment (start 124.797056 73.867056) (end 129.652944 73.867056) (width 1) (layer "F.Cu") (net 1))
 (segment (start 129.652944 73.867056) (end 130.8 72.72) (width 1) (layer "F.Cu") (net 1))
 (segment (start 109 66.8) (end 113.3 66.8) (width 1) (layer "F.Cu") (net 2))
 (segment (start 113.4 66.7) (end 117.3075 66.7) (width 1) (layer "F.Cu") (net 2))
 (segment (start 117.3075 66.7) (end 117.6875 66.32) (width 1) (layer "F.Cu") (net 2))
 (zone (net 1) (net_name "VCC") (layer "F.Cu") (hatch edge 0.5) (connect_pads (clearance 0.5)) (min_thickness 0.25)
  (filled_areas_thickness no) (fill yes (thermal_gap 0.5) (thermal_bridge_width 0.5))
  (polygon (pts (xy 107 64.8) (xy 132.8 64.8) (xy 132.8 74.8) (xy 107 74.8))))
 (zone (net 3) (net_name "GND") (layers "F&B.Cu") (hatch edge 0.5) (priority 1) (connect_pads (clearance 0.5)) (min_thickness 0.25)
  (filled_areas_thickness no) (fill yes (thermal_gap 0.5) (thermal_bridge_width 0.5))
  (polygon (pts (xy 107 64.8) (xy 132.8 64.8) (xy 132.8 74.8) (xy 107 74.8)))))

